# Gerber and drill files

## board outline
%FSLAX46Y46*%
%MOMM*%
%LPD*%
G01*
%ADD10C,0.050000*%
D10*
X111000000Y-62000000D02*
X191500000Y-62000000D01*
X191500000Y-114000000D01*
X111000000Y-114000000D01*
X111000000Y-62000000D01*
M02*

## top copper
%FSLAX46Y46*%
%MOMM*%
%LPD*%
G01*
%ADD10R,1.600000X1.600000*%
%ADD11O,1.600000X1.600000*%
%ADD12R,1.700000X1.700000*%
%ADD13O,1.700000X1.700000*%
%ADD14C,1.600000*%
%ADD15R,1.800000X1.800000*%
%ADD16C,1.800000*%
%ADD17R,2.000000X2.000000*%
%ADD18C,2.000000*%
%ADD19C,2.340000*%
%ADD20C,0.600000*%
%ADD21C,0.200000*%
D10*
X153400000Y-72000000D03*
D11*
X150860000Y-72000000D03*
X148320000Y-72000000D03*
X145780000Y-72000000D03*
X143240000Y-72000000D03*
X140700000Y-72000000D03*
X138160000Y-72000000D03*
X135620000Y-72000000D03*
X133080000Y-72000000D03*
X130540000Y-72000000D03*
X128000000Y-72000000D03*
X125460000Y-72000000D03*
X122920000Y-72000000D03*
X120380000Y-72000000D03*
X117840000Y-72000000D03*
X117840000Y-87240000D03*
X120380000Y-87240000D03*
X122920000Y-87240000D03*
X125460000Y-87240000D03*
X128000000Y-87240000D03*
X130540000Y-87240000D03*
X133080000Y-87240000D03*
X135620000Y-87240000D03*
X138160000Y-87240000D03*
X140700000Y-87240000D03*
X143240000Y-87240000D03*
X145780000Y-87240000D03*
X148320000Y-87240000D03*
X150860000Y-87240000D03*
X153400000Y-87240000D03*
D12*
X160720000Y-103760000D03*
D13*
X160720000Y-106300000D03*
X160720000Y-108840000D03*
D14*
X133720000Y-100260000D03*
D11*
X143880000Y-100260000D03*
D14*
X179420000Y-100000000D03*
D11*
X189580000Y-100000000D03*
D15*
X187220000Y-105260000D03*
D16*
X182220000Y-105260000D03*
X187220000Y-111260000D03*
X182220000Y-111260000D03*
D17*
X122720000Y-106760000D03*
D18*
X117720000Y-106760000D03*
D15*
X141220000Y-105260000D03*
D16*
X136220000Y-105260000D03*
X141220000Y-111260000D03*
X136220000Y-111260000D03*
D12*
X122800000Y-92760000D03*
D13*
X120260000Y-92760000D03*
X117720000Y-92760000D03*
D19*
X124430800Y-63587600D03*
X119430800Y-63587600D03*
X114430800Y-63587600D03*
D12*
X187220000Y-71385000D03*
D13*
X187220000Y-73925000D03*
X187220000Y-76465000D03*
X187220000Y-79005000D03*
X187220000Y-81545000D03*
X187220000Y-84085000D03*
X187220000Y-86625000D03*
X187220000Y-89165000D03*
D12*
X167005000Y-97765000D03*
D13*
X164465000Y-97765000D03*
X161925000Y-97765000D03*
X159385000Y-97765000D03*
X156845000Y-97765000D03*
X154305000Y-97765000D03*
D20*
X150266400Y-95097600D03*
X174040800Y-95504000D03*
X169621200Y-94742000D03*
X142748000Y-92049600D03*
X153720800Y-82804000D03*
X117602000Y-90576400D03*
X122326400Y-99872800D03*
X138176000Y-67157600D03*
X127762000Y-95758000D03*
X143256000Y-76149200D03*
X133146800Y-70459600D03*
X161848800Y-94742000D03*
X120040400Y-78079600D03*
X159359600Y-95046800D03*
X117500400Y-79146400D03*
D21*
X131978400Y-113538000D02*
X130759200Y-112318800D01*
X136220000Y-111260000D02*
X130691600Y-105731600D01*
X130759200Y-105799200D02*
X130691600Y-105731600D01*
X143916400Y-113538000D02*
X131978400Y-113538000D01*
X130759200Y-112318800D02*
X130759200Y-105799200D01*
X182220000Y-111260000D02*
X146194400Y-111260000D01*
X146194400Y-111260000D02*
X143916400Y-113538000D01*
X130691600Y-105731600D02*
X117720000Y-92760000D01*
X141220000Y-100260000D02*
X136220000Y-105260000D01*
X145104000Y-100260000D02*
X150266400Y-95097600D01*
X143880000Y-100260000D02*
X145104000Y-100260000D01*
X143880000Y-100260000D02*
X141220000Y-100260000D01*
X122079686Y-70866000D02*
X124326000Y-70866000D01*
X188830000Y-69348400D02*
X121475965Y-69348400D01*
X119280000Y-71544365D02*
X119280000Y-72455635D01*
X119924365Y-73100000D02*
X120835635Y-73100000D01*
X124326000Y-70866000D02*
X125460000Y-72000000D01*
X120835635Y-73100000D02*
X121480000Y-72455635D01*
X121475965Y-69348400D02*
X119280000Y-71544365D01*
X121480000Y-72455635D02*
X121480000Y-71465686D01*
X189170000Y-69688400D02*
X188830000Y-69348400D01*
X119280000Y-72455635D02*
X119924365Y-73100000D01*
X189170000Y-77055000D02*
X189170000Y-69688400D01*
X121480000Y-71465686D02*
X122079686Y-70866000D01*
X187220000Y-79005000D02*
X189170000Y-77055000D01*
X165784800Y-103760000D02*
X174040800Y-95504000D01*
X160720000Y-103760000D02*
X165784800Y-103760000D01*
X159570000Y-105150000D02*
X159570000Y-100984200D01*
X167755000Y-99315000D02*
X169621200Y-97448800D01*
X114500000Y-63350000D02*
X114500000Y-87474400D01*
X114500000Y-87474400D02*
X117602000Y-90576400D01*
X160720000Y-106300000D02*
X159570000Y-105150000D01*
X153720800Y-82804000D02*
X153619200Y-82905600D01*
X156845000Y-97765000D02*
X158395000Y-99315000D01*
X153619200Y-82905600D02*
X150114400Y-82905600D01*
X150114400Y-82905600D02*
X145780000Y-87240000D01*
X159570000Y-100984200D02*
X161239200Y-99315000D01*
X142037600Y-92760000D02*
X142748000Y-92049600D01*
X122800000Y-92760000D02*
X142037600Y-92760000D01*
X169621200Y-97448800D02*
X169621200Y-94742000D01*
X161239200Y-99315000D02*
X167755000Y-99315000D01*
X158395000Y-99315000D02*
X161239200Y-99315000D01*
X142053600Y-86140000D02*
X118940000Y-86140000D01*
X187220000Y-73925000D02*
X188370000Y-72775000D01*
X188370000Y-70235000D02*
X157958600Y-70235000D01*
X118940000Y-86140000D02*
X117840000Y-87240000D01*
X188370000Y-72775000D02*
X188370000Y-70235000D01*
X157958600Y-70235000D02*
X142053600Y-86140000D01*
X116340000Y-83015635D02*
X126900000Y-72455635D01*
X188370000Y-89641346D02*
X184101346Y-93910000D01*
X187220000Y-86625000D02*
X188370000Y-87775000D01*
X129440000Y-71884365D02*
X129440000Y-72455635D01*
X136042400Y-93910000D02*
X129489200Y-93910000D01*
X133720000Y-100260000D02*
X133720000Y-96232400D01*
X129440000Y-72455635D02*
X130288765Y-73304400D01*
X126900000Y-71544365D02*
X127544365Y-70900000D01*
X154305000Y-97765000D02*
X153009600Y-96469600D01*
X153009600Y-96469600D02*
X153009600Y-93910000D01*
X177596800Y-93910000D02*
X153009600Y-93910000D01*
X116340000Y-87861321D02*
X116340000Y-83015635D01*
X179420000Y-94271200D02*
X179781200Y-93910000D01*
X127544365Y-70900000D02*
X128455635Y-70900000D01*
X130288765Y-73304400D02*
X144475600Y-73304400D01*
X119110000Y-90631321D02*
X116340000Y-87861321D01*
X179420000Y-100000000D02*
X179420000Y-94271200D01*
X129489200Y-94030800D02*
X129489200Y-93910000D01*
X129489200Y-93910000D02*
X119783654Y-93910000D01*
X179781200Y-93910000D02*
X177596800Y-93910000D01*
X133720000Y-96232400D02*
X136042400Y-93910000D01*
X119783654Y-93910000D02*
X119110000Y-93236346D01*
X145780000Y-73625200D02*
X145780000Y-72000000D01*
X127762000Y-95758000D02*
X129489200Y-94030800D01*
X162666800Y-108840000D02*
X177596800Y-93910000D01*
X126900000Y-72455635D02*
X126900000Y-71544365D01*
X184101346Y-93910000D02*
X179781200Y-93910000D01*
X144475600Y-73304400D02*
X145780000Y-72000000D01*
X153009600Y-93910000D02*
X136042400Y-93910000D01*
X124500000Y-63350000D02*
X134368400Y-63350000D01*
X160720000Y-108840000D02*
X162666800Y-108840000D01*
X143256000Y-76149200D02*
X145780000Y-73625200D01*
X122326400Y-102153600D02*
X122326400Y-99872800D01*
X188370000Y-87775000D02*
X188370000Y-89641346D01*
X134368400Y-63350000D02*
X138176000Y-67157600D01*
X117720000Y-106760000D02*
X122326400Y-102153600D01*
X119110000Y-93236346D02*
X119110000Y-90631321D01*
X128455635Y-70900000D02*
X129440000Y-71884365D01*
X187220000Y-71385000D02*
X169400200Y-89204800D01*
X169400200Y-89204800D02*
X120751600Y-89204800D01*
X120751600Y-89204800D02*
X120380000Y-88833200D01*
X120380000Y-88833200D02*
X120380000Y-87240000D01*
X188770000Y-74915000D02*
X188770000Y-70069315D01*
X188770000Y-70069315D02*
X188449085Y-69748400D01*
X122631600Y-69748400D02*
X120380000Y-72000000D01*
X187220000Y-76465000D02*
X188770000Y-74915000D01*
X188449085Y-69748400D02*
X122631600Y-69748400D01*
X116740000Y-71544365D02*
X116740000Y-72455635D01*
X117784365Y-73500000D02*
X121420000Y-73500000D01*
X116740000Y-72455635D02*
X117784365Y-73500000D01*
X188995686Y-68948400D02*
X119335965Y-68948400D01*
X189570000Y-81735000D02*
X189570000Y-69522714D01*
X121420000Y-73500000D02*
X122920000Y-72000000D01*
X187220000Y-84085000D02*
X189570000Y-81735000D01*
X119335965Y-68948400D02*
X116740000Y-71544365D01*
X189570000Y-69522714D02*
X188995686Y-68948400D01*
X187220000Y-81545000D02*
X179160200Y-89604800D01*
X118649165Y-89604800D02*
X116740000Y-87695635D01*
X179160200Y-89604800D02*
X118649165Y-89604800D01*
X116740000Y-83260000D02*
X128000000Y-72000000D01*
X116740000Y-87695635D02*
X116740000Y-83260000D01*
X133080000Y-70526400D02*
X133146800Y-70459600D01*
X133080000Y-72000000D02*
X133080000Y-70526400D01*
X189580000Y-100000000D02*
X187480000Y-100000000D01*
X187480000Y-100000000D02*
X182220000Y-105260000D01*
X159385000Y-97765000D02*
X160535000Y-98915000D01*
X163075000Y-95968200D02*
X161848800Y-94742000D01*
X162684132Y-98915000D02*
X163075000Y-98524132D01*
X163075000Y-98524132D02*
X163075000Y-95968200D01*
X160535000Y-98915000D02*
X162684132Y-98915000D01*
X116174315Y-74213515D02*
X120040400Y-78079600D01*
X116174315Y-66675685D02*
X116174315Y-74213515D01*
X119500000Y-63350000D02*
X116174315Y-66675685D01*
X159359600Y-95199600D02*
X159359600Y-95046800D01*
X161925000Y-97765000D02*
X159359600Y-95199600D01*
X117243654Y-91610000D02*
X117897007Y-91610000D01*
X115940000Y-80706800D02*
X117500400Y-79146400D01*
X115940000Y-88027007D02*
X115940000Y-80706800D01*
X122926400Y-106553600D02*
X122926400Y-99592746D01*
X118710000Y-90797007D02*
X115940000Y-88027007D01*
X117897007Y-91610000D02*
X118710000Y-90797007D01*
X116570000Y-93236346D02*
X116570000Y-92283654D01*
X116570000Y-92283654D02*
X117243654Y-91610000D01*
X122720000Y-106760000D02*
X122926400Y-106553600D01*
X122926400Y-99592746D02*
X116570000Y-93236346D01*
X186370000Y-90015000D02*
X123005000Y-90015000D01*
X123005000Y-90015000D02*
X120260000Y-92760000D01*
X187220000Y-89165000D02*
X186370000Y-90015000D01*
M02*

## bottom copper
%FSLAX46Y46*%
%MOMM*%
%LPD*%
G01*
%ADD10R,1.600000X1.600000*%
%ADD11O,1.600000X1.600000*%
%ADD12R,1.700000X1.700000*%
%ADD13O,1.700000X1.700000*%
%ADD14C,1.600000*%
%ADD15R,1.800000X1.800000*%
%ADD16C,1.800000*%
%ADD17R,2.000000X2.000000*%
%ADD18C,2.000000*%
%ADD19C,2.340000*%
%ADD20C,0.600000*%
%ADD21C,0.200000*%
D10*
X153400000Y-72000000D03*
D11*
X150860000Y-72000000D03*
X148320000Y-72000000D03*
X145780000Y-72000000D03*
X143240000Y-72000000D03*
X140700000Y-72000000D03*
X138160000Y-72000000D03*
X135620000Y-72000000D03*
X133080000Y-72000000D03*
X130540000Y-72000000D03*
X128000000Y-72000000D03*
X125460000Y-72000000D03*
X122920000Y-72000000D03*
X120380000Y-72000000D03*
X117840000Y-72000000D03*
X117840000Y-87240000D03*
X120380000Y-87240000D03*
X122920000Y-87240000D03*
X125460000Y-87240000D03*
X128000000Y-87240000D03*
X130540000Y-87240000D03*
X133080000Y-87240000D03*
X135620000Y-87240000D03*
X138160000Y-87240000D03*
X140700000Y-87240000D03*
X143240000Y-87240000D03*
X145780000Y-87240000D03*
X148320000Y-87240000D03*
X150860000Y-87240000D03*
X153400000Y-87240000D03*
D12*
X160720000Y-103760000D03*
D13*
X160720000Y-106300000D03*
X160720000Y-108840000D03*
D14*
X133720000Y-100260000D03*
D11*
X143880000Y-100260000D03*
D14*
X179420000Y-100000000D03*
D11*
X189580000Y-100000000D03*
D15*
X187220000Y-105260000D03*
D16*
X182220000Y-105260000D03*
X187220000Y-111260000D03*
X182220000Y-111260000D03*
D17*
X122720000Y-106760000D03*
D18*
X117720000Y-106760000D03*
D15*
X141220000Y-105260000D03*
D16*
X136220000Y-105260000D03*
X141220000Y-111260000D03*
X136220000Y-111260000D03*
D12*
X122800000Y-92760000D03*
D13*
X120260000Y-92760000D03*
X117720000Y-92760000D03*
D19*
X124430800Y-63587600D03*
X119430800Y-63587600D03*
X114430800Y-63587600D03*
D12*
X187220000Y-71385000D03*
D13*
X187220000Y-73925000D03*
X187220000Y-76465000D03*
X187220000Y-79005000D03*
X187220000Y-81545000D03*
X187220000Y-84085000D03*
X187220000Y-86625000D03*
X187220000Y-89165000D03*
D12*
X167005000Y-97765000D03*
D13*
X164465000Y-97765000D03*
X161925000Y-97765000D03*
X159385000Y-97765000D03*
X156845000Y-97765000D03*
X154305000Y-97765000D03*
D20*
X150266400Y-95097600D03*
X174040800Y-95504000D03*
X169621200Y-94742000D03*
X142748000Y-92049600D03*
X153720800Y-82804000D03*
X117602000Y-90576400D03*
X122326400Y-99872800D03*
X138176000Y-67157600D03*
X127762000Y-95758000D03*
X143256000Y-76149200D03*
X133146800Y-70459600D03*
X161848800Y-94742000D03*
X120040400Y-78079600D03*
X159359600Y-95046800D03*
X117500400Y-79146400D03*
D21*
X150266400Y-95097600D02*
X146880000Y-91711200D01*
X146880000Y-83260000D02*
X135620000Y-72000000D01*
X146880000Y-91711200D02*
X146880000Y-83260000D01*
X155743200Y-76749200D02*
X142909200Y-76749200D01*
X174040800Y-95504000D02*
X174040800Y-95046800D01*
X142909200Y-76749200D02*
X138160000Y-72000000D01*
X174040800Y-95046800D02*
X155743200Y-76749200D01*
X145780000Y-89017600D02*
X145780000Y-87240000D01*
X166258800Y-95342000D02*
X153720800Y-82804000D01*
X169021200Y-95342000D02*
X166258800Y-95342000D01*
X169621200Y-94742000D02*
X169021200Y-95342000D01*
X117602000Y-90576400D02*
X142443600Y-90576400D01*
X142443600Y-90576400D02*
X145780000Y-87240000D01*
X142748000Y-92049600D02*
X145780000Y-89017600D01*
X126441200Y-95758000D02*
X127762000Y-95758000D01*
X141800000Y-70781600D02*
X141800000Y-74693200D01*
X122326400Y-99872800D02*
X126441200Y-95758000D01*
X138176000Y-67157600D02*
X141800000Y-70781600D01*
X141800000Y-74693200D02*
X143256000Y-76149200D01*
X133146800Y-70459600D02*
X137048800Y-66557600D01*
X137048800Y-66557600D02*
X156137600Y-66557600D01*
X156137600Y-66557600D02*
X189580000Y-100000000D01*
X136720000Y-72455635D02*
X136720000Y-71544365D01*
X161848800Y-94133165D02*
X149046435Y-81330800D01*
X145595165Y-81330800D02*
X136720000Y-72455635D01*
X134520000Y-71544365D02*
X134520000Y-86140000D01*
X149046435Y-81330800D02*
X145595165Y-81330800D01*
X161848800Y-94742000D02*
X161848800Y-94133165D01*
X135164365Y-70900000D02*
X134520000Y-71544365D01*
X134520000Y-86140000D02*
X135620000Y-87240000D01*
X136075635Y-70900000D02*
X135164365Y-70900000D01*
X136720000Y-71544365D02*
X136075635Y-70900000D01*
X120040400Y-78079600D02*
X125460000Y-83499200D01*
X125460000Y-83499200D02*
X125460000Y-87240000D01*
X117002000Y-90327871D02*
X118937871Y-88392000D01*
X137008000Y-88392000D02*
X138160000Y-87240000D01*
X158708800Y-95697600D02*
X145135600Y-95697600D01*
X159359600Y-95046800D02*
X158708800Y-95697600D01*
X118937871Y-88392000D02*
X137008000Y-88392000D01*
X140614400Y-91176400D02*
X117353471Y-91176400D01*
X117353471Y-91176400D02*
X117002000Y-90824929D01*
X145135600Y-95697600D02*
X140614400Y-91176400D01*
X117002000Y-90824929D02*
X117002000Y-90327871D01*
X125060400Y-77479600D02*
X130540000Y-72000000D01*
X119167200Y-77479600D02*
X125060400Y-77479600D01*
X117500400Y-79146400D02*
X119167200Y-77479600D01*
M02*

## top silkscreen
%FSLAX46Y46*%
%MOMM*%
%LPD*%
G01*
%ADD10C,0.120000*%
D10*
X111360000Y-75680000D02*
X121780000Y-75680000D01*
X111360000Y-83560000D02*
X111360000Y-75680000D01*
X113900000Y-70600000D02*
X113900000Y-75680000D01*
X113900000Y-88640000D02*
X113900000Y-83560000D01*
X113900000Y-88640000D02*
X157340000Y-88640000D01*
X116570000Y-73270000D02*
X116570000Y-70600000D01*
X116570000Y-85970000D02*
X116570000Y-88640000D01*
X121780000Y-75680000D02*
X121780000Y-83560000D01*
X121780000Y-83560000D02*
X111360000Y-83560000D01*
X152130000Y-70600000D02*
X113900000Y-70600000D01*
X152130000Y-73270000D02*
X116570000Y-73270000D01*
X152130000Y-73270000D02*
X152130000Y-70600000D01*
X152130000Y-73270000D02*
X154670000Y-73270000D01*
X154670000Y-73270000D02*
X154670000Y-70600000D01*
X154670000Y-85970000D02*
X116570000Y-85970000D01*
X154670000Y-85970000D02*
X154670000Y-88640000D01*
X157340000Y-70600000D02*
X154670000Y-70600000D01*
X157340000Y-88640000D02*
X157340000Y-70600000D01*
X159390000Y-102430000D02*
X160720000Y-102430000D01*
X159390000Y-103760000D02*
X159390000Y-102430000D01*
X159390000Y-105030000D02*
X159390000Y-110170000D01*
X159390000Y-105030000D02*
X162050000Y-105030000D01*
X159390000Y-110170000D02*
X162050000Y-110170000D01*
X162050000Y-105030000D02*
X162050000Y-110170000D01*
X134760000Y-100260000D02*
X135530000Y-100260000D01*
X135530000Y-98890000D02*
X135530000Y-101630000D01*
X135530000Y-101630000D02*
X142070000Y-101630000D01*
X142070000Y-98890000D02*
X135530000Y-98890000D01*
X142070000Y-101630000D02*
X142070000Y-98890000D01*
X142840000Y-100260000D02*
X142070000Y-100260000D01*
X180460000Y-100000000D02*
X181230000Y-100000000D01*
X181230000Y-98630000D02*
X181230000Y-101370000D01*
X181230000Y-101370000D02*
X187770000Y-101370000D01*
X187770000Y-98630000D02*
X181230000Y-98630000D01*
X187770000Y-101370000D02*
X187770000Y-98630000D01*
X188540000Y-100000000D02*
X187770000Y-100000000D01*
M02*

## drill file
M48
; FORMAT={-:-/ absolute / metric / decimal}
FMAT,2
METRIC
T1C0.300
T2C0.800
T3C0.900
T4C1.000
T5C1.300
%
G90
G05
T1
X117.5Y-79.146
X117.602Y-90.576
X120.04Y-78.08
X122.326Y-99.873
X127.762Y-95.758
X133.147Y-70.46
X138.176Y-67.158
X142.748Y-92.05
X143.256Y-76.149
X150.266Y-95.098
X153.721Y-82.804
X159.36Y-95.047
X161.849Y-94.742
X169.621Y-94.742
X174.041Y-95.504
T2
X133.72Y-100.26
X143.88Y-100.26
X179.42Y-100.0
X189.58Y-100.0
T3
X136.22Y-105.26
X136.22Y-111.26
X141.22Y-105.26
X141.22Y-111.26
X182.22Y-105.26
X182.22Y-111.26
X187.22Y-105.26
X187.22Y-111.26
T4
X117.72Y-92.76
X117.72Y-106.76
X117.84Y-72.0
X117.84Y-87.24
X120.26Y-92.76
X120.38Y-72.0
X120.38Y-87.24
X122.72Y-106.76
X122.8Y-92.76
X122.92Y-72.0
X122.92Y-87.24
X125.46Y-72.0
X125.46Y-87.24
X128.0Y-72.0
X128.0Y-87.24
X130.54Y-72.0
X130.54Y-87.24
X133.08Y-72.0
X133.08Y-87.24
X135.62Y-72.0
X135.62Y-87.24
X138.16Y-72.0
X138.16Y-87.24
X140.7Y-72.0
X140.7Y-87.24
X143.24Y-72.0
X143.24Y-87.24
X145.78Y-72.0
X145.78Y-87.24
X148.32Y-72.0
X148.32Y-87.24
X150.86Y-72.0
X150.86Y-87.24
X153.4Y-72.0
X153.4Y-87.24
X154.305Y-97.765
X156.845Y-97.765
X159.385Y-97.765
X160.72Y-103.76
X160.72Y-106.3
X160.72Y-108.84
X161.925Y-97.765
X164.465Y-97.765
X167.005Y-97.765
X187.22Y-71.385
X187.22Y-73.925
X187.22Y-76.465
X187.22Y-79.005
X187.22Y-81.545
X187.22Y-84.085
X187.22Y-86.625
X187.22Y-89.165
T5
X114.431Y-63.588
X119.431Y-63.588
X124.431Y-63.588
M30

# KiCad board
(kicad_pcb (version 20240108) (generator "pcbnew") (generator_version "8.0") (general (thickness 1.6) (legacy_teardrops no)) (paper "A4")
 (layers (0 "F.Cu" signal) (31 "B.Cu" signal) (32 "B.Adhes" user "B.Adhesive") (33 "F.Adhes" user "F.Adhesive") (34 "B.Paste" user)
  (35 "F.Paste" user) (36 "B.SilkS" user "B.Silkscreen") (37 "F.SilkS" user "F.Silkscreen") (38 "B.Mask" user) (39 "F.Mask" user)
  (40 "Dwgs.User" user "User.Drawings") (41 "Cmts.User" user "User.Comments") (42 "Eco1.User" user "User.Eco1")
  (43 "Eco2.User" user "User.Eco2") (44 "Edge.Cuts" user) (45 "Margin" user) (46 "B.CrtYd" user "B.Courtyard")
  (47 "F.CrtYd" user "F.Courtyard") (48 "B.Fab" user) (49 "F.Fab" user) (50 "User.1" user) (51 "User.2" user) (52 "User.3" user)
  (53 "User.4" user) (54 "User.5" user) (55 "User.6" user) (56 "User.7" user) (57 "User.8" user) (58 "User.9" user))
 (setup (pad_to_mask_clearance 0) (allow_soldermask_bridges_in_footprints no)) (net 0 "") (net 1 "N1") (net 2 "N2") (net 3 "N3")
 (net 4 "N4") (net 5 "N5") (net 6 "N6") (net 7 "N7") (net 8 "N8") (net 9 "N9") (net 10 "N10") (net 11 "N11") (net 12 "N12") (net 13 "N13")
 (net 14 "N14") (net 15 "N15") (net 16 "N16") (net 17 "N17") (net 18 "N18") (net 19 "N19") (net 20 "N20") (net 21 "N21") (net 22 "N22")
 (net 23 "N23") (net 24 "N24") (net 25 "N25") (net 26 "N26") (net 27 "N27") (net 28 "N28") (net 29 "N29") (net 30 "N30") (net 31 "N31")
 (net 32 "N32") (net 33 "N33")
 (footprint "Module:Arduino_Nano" (layer "F.Cu") (at 153.4 72 -90)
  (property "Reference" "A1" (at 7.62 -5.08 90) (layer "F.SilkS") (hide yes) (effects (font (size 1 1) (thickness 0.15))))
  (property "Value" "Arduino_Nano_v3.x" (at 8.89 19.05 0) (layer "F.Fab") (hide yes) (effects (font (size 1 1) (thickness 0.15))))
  (fp_line (start 3.68 42.04) (end 3.68 31.62) (stroke (width 0.12) (type solid)) (layer "F.SilkS"))
  (fp_line (start 11.56 42.04) (end 3.68 42.04) (stroke (width 0.12) (type solid)) (layer "F.SilkS"))
  (fp_line (start -1.4 39.5) (end 3.68 39.5) (stroke (width 0.12) (type solid)) (layer "F.SilkS"))
  (fp_line (start 16.64 39.5) (end 11.56 39.5) (stroke (width 0.12) (type solid)) (layer "F.SilkS"))
  (fp_line (start 16.64 39.5) (end 16.64 -3.94) (stroke (width 0.12) (type solid)) (layer "F.SilkS"))
  (fp_line (start 1.27 36.83) (end -1.4 36.83) (stroke (width 0.12) (type solid)) (layer "F.SilkS"))
  (fp_line (start 13.97 36.83) (end 16.64 36.83) (stroke (width 0.12) (type solid)) (layer "F.SilkS"))
  (fp_line (start 3.68 31.62) (end 11.56 31.62) (stroke (width 0.12) (type solid)) (layer "F.SilkS"))
  (fp_line (start 11.56 31.62) (end 11.56 42.04) (stroke (width 0.12) (type solid)) (layer "F.SilkS"))
  (fp_line (start -1.4 1.27) (end -1.4 39.5) (stroke (width 0.12) (type solid)) (layer "F.SilkS"))
  (fp_line (start 1.27 1.27) (end 1.27 36.83) (stroke (width 0.12) (type solid)) (layer "F.SilkS"))
  (fp_line (start 1.27 1.27) (end -1.4 1.27) (stroke (width 0.12) (type solid)) (layer "F.SilkS"))
  (fp_line (start 1.27 1.27) (end 1.27 -1.27) (stroke (width 0.12) (type solid)) (layer "F.SilkS"))
  (fp_line (start 1.27 -1.27) (end -1.4 -1.27) (stroke (width 0.12) (type solid)) (layer "F.SilkS"))
  (fp_line (start 13.97 -1.27) (end 13.97 36.83) (stroke (width 0.12) (type solid)) (layer "F.SilkS"))
  (fp_line (start 13.97 -1.27) (end 16.64 -1.27) (stroke (width 0.12) (type solid)) (layer "F.SilkS"))
  (fp_line (start -1.4 -3.94) (end -1.4 -1.27) (stroke (width 0.12) (type solid)) (layer "F.SilkS"))
  (fp_line (start 16.64 -3.94) (end -1.4 -3.94) (stroke (width 0.12) (type solid)) (layer "F.SilkS"))
  (pad "1" thru_hole rect (at 0 0 270) (size 1.6 1.6) (drill 1) (layers "*.Cu" "*.Mask") (remove_unused_layers no) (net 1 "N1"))
  (pad "2" thru_hole oval (at 0 2.54 270) (size 1.6 1.6) (drill 1) (layers "*.Cu" "*.Mask") (remove_unused_layers no) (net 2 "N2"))
  (pad "3" thru_hole oval (at 0 5.08 270) (size 1.6 1.6) (drill 1) (layers "*.Cu" "*.Mask") (remove_unused_layers no) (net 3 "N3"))
  (pad "4" thru_hole oval (at 0 7.62 270) (size 1.6 1.6) (drill 1) (layers "*.Cu" "*.Mask") (remove_unused_layers no) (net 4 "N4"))
  (pad "5" thru_hole oval (at 0 10.16 270) (size 1.6 1.6) (drill 1) (layers "*.Cu" "*.Mask") (remove_unused_layers no) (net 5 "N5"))
  (pad "6" thru_hole oval (at 0 12.7 270) (size 1.6 1.6) (drill 1) (layers "*.Cu" "*.Mask") (remove_unused_layers no) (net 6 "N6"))
  (pad "7" thru_hole oval (at 0 15.24 270) (size 1.6 1.6) (drill 1) (layers "*.Cu" "*.Mask") (remove_unused_layers no) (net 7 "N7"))
  (pad "8" thru_hole oval (at 0 17.78 270) (size 1.6 1.6) (drill 1) (layers "*.Cu" "*.Mask") (remove_unused_layers no) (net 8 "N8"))
  (pad "9" thru_hole oval (at 0 20.32 270) (size 1.6 1.6) (drill 1) (layers "*.Cu" "*.Mask") (remove_unused_layers no) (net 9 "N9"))
  (pad "10" thru_hole oval (at 0 22.86 270) (size 1.6 1.6) (drill 1) (layers "*.Cu" "*.Mask") (remove_unused_layers no) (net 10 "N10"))
  (pad "11" thru_hole oval (at 0 25.4 270) (size 1.6 1.6) (drill 1) (layers "*.Cu" "*.Mask") (remove_unused_layers no) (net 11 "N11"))
  (pad "12" thru_hole oval (at 0 27.94 270) (size 1.6 1.6) (drill 1) (layers "*.Cu" "*.Mask") (remove_unused_layers no) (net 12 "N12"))
  (pad "13" thru_hole oval (at 0 30.48 270) (size 1.6 1.6) (drill 1) (layers "*.Cu" "*.Mask") (remove_unused_layers no) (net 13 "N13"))
  (pad "14" thru_hole oval (at 0 33.02 270) (size 1.6 1.6) (drill 1) (layers "*.Cu" "*.Mask") (remove_unused_layers no) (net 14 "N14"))
  (pad "15" thru_hole oval (at 0 35.56 270) (size 1.6 1.6) (drill 1) (layers "*.Cu" "*.Mask") (remove_unused_layers no) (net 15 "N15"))
  (pad "16" thru_hole oval (at 15.24 35.56 270) (size 1.6 1.6) (drill 1) (layers "*.Cu" "*.Mask") (remove_unused_layers no) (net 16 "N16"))
  (pad "17" thru_hole oval (at 15.24 33.02 270) (size 1.6 1.6) (drill 1) (layers "*.Cu" "*.Mask") (remove_unused_layers no) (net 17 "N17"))
  (pad "18" thru_hole oval (at 15.24 30.48 270) (size 1.6 1.6) (drill 1) (layers "*.Cu" "*.Mask") (remove_unused_layers no) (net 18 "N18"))
  (pad "19" thru_hole oval (at 15.24 27.94 270) (size 1.6 1.6) (drill 1) (layers "*.Cu" "*.Mask") (remove_unused_layers no) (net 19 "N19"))
  (pad "20" thru_hole oval (at 15.24 25.4 270) (size 1.6 1.6) (drill 1) (layers "*.Cu" "*.Mask") (remove_unused_layers no) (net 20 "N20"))
  (pad "21" thru_hole oval (at 15.24 22.86 270) (size 1.6 1.6) (drill 1) (layers "*.Cu" "*.Mask") (remove_unused_layers no) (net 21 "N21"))
  (pad "22" thru_hole oval (at 15.24 20.32 270) (size 1.6 1.6) (drill 1) (layers "*.Cu" "*.Mask") (remove_unused_layers no) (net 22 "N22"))
  (pad "23" thru_hole oval (at 15.24 17.78 270) (size 1.6 1.6) (drill 1) (layers "*.Cu" "*.Mask") (remove_unused_layers no) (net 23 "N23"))
  (pad "24" thru_hole oval (at 15.24 15.24 270) (size 1.6 1.6) (drill 1) (layers "*.Cu" "*.Mask") (remove_unused_layers no) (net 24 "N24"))
  (pad "25" thru_hole oval (at 15.24 12.7 270) (size 1.6 1.6) (drill 1) (layers "*.Cu" "*.Mask") (remove_unused_layers no) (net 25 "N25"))
  (pad "26" thru_hole oval (at 15.24 10.16 270) (size 1.6 1.6) (drill 1) (layers "*.Cu" "*.Mask") (remove_unused_layers no) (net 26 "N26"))
  (pad "27" thru_hole oval (at 15.24 7.62 270) (size 1.6 1.6) (drill 1) (layers "*.Cu" "*.Mask") (remove_unused_layers no) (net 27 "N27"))
  (pad "28" thru_hole oval (at 15.24 5.08 270) (size 1.6 1.6) (drill 1) (layers "*.Cu" "*.Mask") (remove_unused_layers no) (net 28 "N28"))
  (pad "29" thru_hole oval (at 15.24 2.54 270) (size 1.6 1.6) (drill 1) (layers "*.Cu" "*.Mask") (remove_unused_layers no) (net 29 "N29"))
  (pad "30" thru_hole oval (at 15.24 0 270) (size 1.6 1.6) (drill 1) (layers "*.Cu" "*.Mask") (remove_unused_layers no) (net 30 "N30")))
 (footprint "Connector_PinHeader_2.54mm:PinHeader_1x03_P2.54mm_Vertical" (layer "F.Cu") (at 160.72 103.76)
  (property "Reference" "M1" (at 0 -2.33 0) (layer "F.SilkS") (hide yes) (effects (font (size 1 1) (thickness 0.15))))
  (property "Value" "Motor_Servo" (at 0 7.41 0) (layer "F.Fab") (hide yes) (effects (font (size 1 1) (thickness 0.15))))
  (fp_line (start -1.33 -1.33) (end 0 -1.33) (stroke (width 0.12) (type solid)) (layer "F.SilkS"))
  (fp_line (start -1.33 0) (end -1.33 -1.33) (stroke (width 0.12) (type solid)) (layer "F.SilkS"))
  (fp_line (start -1.33 1.27) (end -1.33 6.41) (stroke (width 0.12) (type solid)) (layer "F.SilkS"))
  (fp_line (start -1.33 1.27) (end 1.33 1.27) (stroke (width 0.12) (type solid)) (layer "F.SilkS"))
  (fp_line (start -1.33 6.41) (end 1.33 6.41) (stroke (width 0.12) (type solid)) (layer "F.SilkS"))
  (fp_line (start 1.33 1.27) (end 1.33 6.41) (stroke (width 0.12) (type solid)) (layer "F.SilkS"))
  (pad "1" thru_hole rect (at 0 0) (size 1.7 1.7) (drill 1) (layers "*.Cu" "*.Mask") (remove_unused_layers no) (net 7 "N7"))
  (pad "2" thru_hole oval (at 0 2.54) (size 1.7 1.7) (drill 1) (layers "*.Cu" "*.Mask") (remove_unused_layers no) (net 27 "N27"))
  (pad "3" thru_hole oval (at 0 5.08) (size 1.7 1.7) (drill 1) (layers "*.Cu" "*.Mask") (remove_unused_layers no) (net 4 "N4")))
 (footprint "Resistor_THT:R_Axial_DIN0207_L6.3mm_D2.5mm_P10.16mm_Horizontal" (layer "F.Cu") (at 133.72 100.26)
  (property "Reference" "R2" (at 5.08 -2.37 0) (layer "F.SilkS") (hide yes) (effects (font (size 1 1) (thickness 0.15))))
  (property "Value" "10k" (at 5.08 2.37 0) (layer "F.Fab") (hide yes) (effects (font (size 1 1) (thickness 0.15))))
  (fp_line (start 1.04 0) (end 1.81 0) (stroke (width 0.12) (type solid)) (layer "F.SilkS"))
  (fp_line (start 1.81 -1.37) (end 1.81 1.37) (stroke (width 0.12) (type solid)) (layer "F.SilkS"))
  (fp_line (start 1.81 1.37) (end 8.35 1.37) (stroke (width 0.12) (type solid)) (layer "F.SilkS"))
  (fp_line (start 8.35 -1.37) (end 1.81 -1.37) (stroke (width 0.12) (type solid)) (layer "F.SilkS"))
  (fp_line (start 8.35 1.37) (end 8.35 -1.37) (stroke (width 0.12) (type solid)) (layer "F.SilkS"))
  (fp_line (start 9.12 0) (end 8.35 0) (stroke (width 0.12) (type solid)) (layer "F.SilkS"))
  (pad "1" thru_hole circle (at 0 0) (size 1.6 1.6) (drill 0.8) (layers "*.Cu" "*.Mask") (remove_unused_layers no) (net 4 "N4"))
  (pad "2" thru_hole oval (at 10.16 0) (size 1.6 1.6) (drill 0.8) (layers "*.Cu" "*.Mask") (remove_unused_layers no) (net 8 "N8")))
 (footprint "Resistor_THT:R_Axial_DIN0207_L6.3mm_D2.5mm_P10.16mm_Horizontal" (layer "F.Cu") (at 179.42 100)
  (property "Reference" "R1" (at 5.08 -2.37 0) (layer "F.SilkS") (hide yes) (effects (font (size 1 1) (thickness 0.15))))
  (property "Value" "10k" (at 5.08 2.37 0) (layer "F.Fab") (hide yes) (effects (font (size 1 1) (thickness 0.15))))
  (fp_line (start 1.04 0) (end 1.81 0) (stroke (width 0.12) (type solid)) (layer "F.SilkS"))
  (fp_line (start 1.81 -1.37) (end 1.81 1.37) (stroke (width 0.12) (type solid)) (layer "F.SilkS"))
  (fp_line (start 1.81 1.37) (end 8.35 1.37) (stroke (width 0.12) (type solid)) (layer "F.SilkS"))
  (fp_line (start 8.35 -1.37) (end 1.81 -1.37) (stroke (width 0.12) (type solid)) (layer "F.SilkS"))
  (fp_line (start 8.35 1.37) (end 8.35 -1.37) (stroke (width 0.12) (type solid)) (layer "F.SilkS"))
  (fp_line (start 9.12 0) (end 8.35 0) (stroke (width 0.12) (type solid)) (layer "F.SilkS"))
  (pad "1" thru_hole circle (at 0 0) (size 1.6 1.6) (drill 0.8) (layers "*.Cu" "*.Mask") (remove_unused_layers no) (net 4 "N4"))
  (pad "2" thru_hole oval (at 10.16 0) (size 1.6 1.6) (drill 0.8) (layers "*.Cu" "*.Mask") (remove_unused_layers no) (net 9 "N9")))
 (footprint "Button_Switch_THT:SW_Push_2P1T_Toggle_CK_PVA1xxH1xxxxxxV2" (layer "B.Cu") (at 187.22 105.26 180)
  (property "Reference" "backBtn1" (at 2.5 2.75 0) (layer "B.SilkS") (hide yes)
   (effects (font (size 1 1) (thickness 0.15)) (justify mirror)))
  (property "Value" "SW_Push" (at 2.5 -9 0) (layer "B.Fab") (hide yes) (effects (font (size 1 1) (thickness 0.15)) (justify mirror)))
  (pad "1" thru_hole rect (at 0 0 180) (size 1.8 1.8) (drill 0.9) (layers "*.Cu" "*.Mask") (remove_unused_layers no) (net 27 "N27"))
  (pad "2" thru_hole circle (at 5 0 180) (size 1.8 1.8) (drill 0.9) (layers "*.Cu" "*.Mask") (remove_unused_layers no) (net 9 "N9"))
  (pad "3" thru_hole circle (at 0 -6 180) (size 1.8 1.8) (drill 0.9) (layers "*.Cu" "*.Mask") (remove_unused_layers no))
  (pad "4" thru_hole circle (at 5 -6 180) (size 1.8 1.8) (drill 0.9) (layers "*.Cu" "*.Mask") (remove_unused_layers no)))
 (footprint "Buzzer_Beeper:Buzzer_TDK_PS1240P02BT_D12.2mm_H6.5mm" (layer "B.Cu") (at 122.72 106.76 180)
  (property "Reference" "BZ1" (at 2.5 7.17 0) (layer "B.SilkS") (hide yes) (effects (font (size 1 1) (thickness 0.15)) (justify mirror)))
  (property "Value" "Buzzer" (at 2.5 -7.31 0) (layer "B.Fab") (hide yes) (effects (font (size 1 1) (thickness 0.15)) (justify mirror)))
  (pad "1" thru_hole rect (at 0 0 180) (size 2 2) (drill 1) (layers "*.Cu" "*.Mask") (remove_unused_layers no) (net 10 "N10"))
  (pad "2" thru_hole circle (at 5 0 180) (size 2 2) (drill 1) (layers "*.Cu" "*.Mask") (remove_unused_layers no) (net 4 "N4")))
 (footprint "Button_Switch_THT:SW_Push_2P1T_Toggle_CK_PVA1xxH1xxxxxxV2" (layer "B.Cu") (at 141.22 105.26 180)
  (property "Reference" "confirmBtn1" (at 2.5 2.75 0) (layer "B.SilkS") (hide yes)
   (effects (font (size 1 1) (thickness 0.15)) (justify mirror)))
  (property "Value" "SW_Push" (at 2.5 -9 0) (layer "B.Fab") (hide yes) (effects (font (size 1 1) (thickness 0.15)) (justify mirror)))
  (pad "1" thru_hole rect (at 0 0 180) (size 1.8 1.8) (drill 0.9) (layers "*.Cu" "*.Mask") (remove_unused_layers no) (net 27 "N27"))
  (pad "2" thru_hole circle (at 5 0 180) (size 1.8 1.8) (drill 0.9) (layers "*.Cu" "*.Mask") (remove_unused_layers no) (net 8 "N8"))
  (pad "3" thru_hole circle (at 0 -6 180) (size 1.8 1.8) (drill 0.9) (layers "*.Cu" "*.Mask") (remove_unused_layers no))
  (pad "4" thru_hole circle (at 5 -6 180) (size 1.8 1.8) (drill 0.9) (layers "*.Cu" "*.Mask") (remove_unused_layers no)))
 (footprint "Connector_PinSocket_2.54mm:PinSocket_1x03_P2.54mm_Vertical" (layer "B.Cu") (at 122.8 92.76 90)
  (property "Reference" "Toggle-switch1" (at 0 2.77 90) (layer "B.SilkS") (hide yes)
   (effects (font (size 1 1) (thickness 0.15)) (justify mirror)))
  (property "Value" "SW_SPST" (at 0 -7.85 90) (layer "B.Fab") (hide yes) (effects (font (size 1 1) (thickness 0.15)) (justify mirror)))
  (pad "1" thru_hole rect (at 0 0 90) (size 1.7 1.7) (drill 1) (layers "*.Cu" "*.Mask") (remove_unused_layers no) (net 27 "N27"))
  (pad "2" thru_hole oval (at 0 -2.54 90) (size 1.7 1.7) (drill 1) (layers "*.Cu" "*.Mask") (remove_unused_layers no) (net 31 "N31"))
  (pad "3" thru_hole oval (at 0 -5.08 90) (size 1.7 1.7) (drill 1) (layers "*.Cu" "*.Mask") (remove_unused_layers no)))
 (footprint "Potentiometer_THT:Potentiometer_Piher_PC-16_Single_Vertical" (layer "B.Cu") (at 124.4308 63.5876 -90)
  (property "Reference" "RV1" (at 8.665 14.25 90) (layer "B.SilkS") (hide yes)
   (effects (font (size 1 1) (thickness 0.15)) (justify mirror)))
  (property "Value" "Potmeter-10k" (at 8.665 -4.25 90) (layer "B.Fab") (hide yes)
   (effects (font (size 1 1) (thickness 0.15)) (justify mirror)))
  (pad "1" thru_hole circle (at 0 0 270) (size 2.34 2.34) (drill 1.3) (layers "*.Cu" "*.Mask") (remove_unused_layers no) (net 4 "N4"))
  (pad "2" thru_hole circle (at 0 5 270) (size 2.34 2.34) (drill 1.3) (layers "*.Cu" "*.Mask") (remove_unused_layers no) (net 19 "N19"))
  (pad "3" thru_hole circle (at 0 10 270) (size 2.34 2.34) (drill 1.3) (layers "*.Cu" "*.Mask") (remove_unused_layers no) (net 27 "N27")))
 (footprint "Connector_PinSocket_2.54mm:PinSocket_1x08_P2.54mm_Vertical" (layer "B.Cu") (at 187.22 71.385 180)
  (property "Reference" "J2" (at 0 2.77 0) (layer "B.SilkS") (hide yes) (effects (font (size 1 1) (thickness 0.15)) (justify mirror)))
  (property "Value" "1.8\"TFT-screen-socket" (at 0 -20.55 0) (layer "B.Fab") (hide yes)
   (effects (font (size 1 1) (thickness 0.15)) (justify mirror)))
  (pad "1" thru_hole rect (at 0 0 180) (size 1.7 1.7) (drill 1) (layers "*.Cu" "*.Mask") (remove_unused_layers no) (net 17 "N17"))
  (pad "2" thru_hole oval (at 0 -2.54 180) (size 1.7 1.7) (drill 1) (layers "*.Cu" "*.Mask") (remove_unused_layers no) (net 16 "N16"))
  (pad "3" thru_hole oval (at 0 -5.08 180) (size 1.7 1.7) (drill 1) (layers "*.Cu" "*.Mask") (remove_unused_layers no) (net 14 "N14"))
  (pad "4" thru_hole oval (at 0 -7.62 180) (size 1.7 1.7) (drill 1) (layers "*.Cu" "*.Mask") (remove_unused_layers no) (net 12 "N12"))
  (pad "5" thru_hole oval (at 0 -10.16 180) (size 1.7 1.7) (drill 1) (layers "*.Cu" "*.Mask") (remove_unused_layers no) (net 11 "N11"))
  (pad "6" thru_hole oval (at 0 -12.7 180) (size 1.7 1.7) (drill 1) (layers "*.Cu" "*.Mask") (remove_unused_layers no) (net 13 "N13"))
  (pad "7" thru_hole oval (at 0 -15.24 180) (size 1.7 1.7) (drill 1) (layers "*.Cu" "*.Mask") (remove_unused_layers no) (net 4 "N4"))
  (pad "8" thru_hole oval (at 0 -17.78 180) (size 1.7 1.7) (drill 1) (layers "*.Cu" "*.Mask") (remove_unused_layers no) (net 31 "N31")))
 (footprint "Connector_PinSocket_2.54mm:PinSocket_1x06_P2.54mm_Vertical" (layer "B.Cu") (at 167.005 97.765 90)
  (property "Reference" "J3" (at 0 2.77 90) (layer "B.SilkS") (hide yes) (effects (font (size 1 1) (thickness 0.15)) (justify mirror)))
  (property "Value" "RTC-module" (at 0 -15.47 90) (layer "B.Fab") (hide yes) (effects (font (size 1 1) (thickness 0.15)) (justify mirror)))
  (pad "1" thru_hole rect (at 0 0 90) (size 1.7 1.7) (drill 1) (layers "*.Cu" "*.Mask") (remove_unused_layers no) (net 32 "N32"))
  (pad "2" thru_hole oval (at 0 -2.54 90) (size 1.7 1.7) (drill 1) (layers "*.Cu" "*.Mask") (remove_unused_layers no) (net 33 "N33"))
  (pad "3" thru_hole oval (at 0 -5.08 90) (size 1.7 1.7) (drill 1) (layers "*.Cu" "*.Mask") (remove_unused_layers no) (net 24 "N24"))
  (pad "4" thru_hole oval (at 0 -7.62 90) (size 1.7 1.7) (drill 1) (layers "*.Cu" "*.Mask") (remove_unused_layers no) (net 23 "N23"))
  (pad "5" thru_hole oval (at 0 -10.16 90) (size 1.7 1.7) (drill 1) (layers "*.Cu" "*.Mask") (remove_unused_layers no) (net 27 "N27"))
  (pad "6" thru_hole oval (at 0 -12.7 90) (size 1.7 1.7) (drill 1) (layers "*.Cu" "*.Mask") (remove_unused_layers no) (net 4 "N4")))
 (gr_rect (start 111 62) (end 191.5 114) (stroke (width 0.05) (type default)) (fill none) (layer "Edge.Cuts"))
 (segment (start 131.9784 113.538) (end 130.7592 112.3188) (width 0.2) (layer "F.Cu") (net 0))
 (segment (start 136.22 111.26) (end 130.6916 105.7316) (width 0.2) (layer "F.Cu") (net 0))
 (segment (start 130.7592 105.7992) (end 130.6916 105.7316) (width 0.2) (layer "F.Cu") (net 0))
 (segment (start 143.9164 113.538) (end 131.9784 113.538) (width 0.2) (layer "F.Cu") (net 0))
 (segment (start 130.7592 112.3188) (end 130.7592 105.7992) (width 0.2) (layer "F.Cu") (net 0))
 (segment (start 182.22 111.26) (end 146.1944 111.26) (width 0.2) (layer "F.Cu") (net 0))
 (segment (start 146.1944 111.26) (end 143.9164 113.538) (width 0.2) (layer "F.Cu") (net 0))
 (segment (start 130.6916 105.7316) (end 117.72 92.76) (width 0.2) (layer "F.Cu") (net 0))
 (segment (start 141.22 100.26) (end 136.22 105.26) (width 0.2) (layer "F.Cu") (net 8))
 (segment (start 145.104 100.26) (end 150.2664 95.0976) (width 0.2) (layer "F.Cu") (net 8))
 (segment (start 143.88 100.26) (end 145.104 100.26) (width 0.2) (layer "F.Cu") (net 8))
 (segment (start 143.88 100.26) (end 141.22 100.26) (width 0.2) (layer "F.Cu") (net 8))
 (via (at 150.2664 95.0976) (size 0.6) (drill 0.3) (layers "F.Cu" "B.Cu") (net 8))
 (segment (start 150.2664 95.0976) (end 146.88 91.7112) (width 0.2) (layer "B.Cu") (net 8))
 (segment (start 146.88 83.26) (end 135.62 72) (width 0.2) (layer "B.Cu") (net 8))
 (segment (start 146.88 91.7112) (end 146.88 83.26) (width 0.2) (layer "B.Cu") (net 8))
 (segment (start 122.079686 70.866) (end 124.326 70.866) (width 0.2) (layer "F.Cu") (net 12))
 (segment (start 188.83 69.3484) (end 121.475965 69.3484) (width 0.2) (layer "F.Cu") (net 12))
 (segment (start 119.28 71.544365) (end 119.28 72.455635) (width 0.2) (layer "F.Cu") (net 12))
 (segment (start 119.924365 73.1) (end 120.835635 73.1) (width 0.2) (layer "F.Cu") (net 12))
 (segment (start 124.326 70.866) (end 125.46 72) (width 0.2) (layer "F.Cu") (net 12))
 (segment (start 120.835635 73.1) (end 121.48 72.455635) (width 0.2) (layer "F.Cu") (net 12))
 (segment (start 121.475965 69.3484) (end 119.28 71.544365) (width 0.2) (layer "F.Cu") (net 12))
 (segment (start 121.48 72.455635) (end 121.48 71.465686) (width 0.2) (layer "F.Cu") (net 12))
 (segment (start 189.17 69.6884) (end 188.83 69.3484) (width 0.2) (layer "F.Cu") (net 12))
 (segment (start 119.28 72.455635) (end 119.924365 73.1) (width 0.2) (layer "F.Cu") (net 12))
 (segment (start 189.17 77.055) (end 189.17 69.6884) (width 0.2) (layer "F.Cu") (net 12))
 (segment (start 121.48 71.465686) (end 122.079686 70.866) (width 0.2) (layer "F.Cu") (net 12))
 (segment (start 187.22 79.005) (end 189.17 77.055) (width 0.2) (layer "F.Cu") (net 12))
 (segment (start 165.7848 103.76) (end 174.0408 95.504) (width 0.2) (layer "F.Cu") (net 7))
 (segment (start 160.72 103.76) (end 165.7848 103.76) (width 0.2) (layer "F.Cu") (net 7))
 (via (at 174.0408 95.504) (size 0.6) (drill 0.3) (layers "F.Cu" "B.Cu") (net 7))
 (segment (start 155.7432 76.7492) (end 142.9092 76.7492) (width 0.2) (layer "B.Cu") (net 7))
 (segment (start 174.0408 95.504) (end 174.0408 95.0468) (width 0.2) (layer "B.Cu") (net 7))
 (segment (start 142.9092 76.7492) (end 138.16 72) (width 0.2) (layer "B.Cu") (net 7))
 (segment (start 174.0408 95.0468) (end 155.7432 76.7492) (width 0.2) (layer "B.Cu") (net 7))
 (segment (start 159.57 105.15) (end 159.57 100.9842) (width 0.2) (layer "F.Cu") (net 27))
 (segment (start 167.755 99.315) (end 169.6212 97.4488) (width 0.2) (layer "F.Cu") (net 27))
 (segment (start 114.5 63.35) (end 114.5 87.4744) (width 0.2) (layer "F.Cu") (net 27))
 (segment (start 114.5 87.4744) (end 117.602 90.5764) (width 0.2) (layer "F.Cu") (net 27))
 (segment (start 160.72 106.3) (end 159.57 105.15) (width 0.2) (layer "F.Cu") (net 27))
 (segment (start 153.7208 82.804) (end 153.6192 82.9056) (width 0.2) (layer "F.Cu") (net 27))
 (segment (start 156.845 97.765) (end 158.395 99.315) (width 0.2) (layer "F.Cu") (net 27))
 (segment (start 153.6192 82.9056) (end 150.1144 82.9056) (width 0.2) (layer "F.Cu") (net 27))
 (segment (start 150.1144 82.9056) (end 145.78 87.24) (width 0.2) (layer "F.Cu") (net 27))
 (segment (start 159.57 100.9842) (end 161.2392 99.315) (width 0.2) (layer "F.Cu") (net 27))
 (segment (start 142.0376 92.76) (end 142.748 92.0496) (width 0.2) (layer "F.Cu") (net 27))
 (segment (start 122.8 92.76) (end 142.0376 92.76) (width 0.2) (layer "F.Cu") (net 27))
 (segment (start 169.6212 97.4488) (end 169.6212 94.742) (width 0.2) (layer "F.Cu") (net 27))
 (segment (start 161.2392 99.315) (end 167.755 99.315) (width 0.2) (layer "F.Cu") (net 27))
 (segment (start 158.395 99.315) (end 161.2392 99.315) (width 0.2) (layer "F.Cu") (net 27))
 (via (at 169.6212 94.742) (size 0.6) (drill 0.3) (layers "F.Cu" "B.Cu") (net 27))
 (via (at 142.748 92.0496) (size 0.6) (drill 0.3) (layers "F.Cu" "B.Cu") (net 27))
 (via (at 153.7208 82.804) (size 0.6) (drill 0.3) (layers "F.Cu" "B.Cu") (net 27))
 (via (at 117.602 90.5764) (size 0.6) (drill 0.3) (layers "F.Cu" "B.Cu") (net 27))
 (segment (start 145.78 89.0176) (end 145.78 87.24) (width 0.2) (layer "B.Cu") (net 27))
 (segment (start 166.2588 95.342) (end 153.7208 82.804) (width 0.2) (layer "B.Cu") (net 27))
 (segment (start 169.0212 95.342) (end 166.2588 95.342) (width 0.2) (layer "B.Cu") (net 27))
 (segment (start 169.6212 94.742) (end 169.0212 95.342) (width 0.2) (layer "B.Cu") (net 27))
 (segment (start 117.602 90.5764) (end 142.4436 90.5764) (width 0.2) (layer "B.Cu") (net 27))
 (segment (start 142.4436 90.5764) (end 145.78 87.24) (width 0.2) (layer "B.Cu") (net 27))
 (segment (start 142.748 92.0496) (end 145.78 89.0176) (width 0.2) (layer "B.Cu") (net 27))
 (segment (start 142.0536 86.14) (end 118.94 86.14) (width 0.2) (layer "F.Cu") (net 16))
 (segment (start 187.22 73.925) (end 188.37 72.775) (width 0.2) (layer "F.Cu") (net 16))
 (segment (start 188.37 70.235) (end 157.9586 70.235) (width 0.2) (layer "F.Cu") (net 16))
 (segment (start 118.94 86.14) (end 117.84 87.24) (width 0.2) (layer "F.Cu") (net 16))
 (segment (start 188.37 72.775) (end 188.37 70.235) (width 0.2) (layer "F.Cu") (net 16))
 (segment (start 157.9586 70.235) (end 142.0536 86.14) (width 0.2) (layer "F.Cu") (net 16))
 (segment (start 116.34 83.015635) (end 126.9 72.455635) (width 0.2) (layer "F.Cu") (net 4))
 (segment (start 188.37 89.641346) (end 184.101346 93.91) (width 0.2) (layer "F.Cu") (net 4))
 (segment (start 187.22 86.625) (end 188.37 87.775) (width 0.2) (layer "F.Cu") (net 4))
 (segment (start 129.44 71.884365) (end 129.44 72.455635) (width 0.2) (layer "F.Cu") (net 4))
 (segment (start 136.0424 93.91) (end 129.4892 93.91) (width 0.2) (layer "F.Cu") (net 4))
 (segment (start 133.72 100.26) (end 133.72 96.2324) (width 0.2) (layer "F.Cu") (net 4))
 (segment (start 129.44 72.455635) (end 130.288765 73.3044) (width 0.2) (layer "F.Cu") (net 4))
 (segment (start 126.9 71.544365) (end 127.544365 70.9) (width 0.2) (layer "F.Cu") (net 4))
 (segment (start 154.305 97.765) (end 153.0096 96.4696) (width 0.2) (layer "F.Cu") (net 4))
 (segment (start 153.0096 96.4696) (end 153.0096 93.91) (width 0.2) (layer "F.Cu") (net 4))
 (segment (start 177.5968 93.91) (end 153.0096 93.91) (width 0.2) (layer "F.Cu") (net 4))
 (segment (start 116.34 87.861321) (end 116.34 83.015635) (width 0.2) (layer "F.Cu") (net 4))
 (segment (start 179.42 94.2712) (end 179.7812 93.91) (width 0.2) (layer "F.Cu") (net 4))
 (segment (start 127.544365 70.9) (end 128.455635 70.9) (width 0.2) (layer "F.Cu") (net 4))
 (segment (start 130.288765 73.3044) (end 144.4756 73.3044) (width 0.2) (layer "F.Cu") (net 4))
 (segment (start 119.11 90.631321) (end 116.34 87.861321) (width 0.2) (layer "F.Cu") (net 4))
 (segment (start 179.42 100) (end 179.42 94.2712) (width 0.2) (layer "F.Cu") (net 4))
 (segment (start 129.4892 94.0308) (end 129.4892 93.91) (width 0.2) (layer "F.Cu") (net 4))
 (segment (start 129.4892 93.91) (end 119.783654 93.91) (width 0.2) (layer "F.Cu") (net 4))
 (segment (start 179.7812 93.91) (end 177.5968 93.91) (width 0.2) (layer "F.Cu") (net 4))
 (segment (start 133.72 96.2324) (end 136.0424 93.91) (width 0.2) (layer "F.Cu") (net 4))
 (segment (start 119.783654 93.91) (end 119.11 93.236346) (width 0.2) (layer "F.Cu") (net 4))
 (segment (start 145.78 73.6252) (end 145.78 72) (width 0.2) (layer "F.Cu") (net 4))
 (segment (start 127.762 95.758) (end 129.4892 94.0308) (width 0.2) (layer "F.Cu") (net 4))
 (segment (start 162.6668 108.84) (end 177.5968 93.91) (width 0.2) (layer "F.Cu") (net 4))
 (segment (start 126.9 72.455635) (end 126.9 71.544365) (width 0.2) (layer "F.Cu") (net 4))
 (segment (start 184.101346 93.91) (end 179.7812 93.91) (width 0.2) (layer "F.Cu") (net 4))
 (segment (start 144.4756 73.3044) (end 145.78 72) (width 0.2) (layer "F.Cu") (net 4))
 (segment (start 153.0096 93.91) (end 136.0424 93.91) (width 0.2) (layer "F.Cu") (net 4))
 (segment (start 124.5 63.35) (end 134.3684 63.35) (width 0.2) (layer "F.Cu") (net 4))
 (segment (start 160.72 108.84) (end 162.6668 108.84) (width 0.2) (layer "F.Cu") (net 4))
 (segment (start 143.256 76.1492) (end 145.78 73.6252) (width 0.2) (layer "F.Cu") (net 4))
 (segment (start 122.3264 102.1536) (end 122.3264 99.8728) (width 0.2) (layer "F.Cu") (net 4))
 (segment (start 188.37 87.775) (end 188.37 89.641346) (width 0.2) (layer "F.Cu") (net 4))
 (segment (start 134.3684 63.35) (end 138.176 67.1576) (width 0.2) (layer "F.Cu") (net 4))
 (segment (start 117.72 106.76) (end 122.3264 102.1536) (width 0.2) (layer "F.Cu") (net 4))
 (segment (start 119.11 93.236346) (end 119.11 90.631321) (width 0.2) (layer "F.Cu") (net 4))
 (segment (start 128.455635 70.9) (end 129.44 71.884365) (width 0.2) (layer "F.Cu") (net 4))
 (via (at 122.3264 99.8728) (size 0.6) (drill 0.3) (layers "F.Cu" "B.Cu") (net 4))
 (via (at 138.176 67.1576) (size 0.6) (drill 0.3) (layers "F.Cu" "B.Cu") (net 4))
 (via (at 127.762 95.758) (size 0.6) (drill 0.3) (layers "F.Cu" "B.Cu") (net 4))
 (via (at 143.256 76.1492) (size 0.6) (drill 0.3) (layers "F.Cu" "B.Cu") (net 4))
 (segment (start 126.4412 95.758) (end 127.762 95.758) (width 0.2) (layer "B.Cu") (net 4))
 (segment (start 141.8 70.7816) (end 141.8 74.6932) (width 0.2) (layer "B.Cu") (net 4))
 (segment (start 122.3264 99.8728) (end 126.4412 95.758) (width 0.2) (layer "B.Cu") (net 4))
 (segment (start 138.176 67.1576) (end 141.8 70.7816) (width 0.2) (layer "B.Cu") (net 4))
 (segment (start 141.8 74.6932) (end 143.256 76.1492) (width 0.2) (layer "B.Cu") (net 4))
 (segment (start 187.22 71.385) (end 169.4002 89.2048) (width 0.2) (layer "F.Cu") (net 17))
 (segment (start 169.4002 89.2048) (end 120.7516 89.2048) (width 0.2) (layer "F.Cu") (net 17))
 (segment (start 120.7516 89.2048) (end 120.38 88.8332) (width 0.2) (layer "F.Cu") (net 17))
 (segment (start 120.38 88.8332) (end 120.38 87.24) (width 0.2) (layer "F.Cu") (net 17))
 (segment (start 188.77 74.915) (end 188.77 70.069315) (width 0.2) (layer "F.Cu") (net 14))
 (segment (start 188.77 70.069315) (end 188.449085 69.7484) (width 0.2) (layer "F.Cu") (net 14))
 (segment (start 122.6316 69.7484) (end 120.38 72) (width 0.2) (layer "F.Cu") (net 14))
 (segment (start 187.22 76.465) (end 188.77 74.915) (width 0.2) (layer "F.Cu") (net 14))
 (segment (start 188.449085 69.7484) (end 122.6316 69.7484) (width 0.2) (layer "F.Cu") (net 14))
 (segment (start 116.74 71.544365) (end 116.74 72.455635) (width 0.2) (layer "F.Cu") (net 13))
 (segment (start 117.784365 73.5) (end 121.42 73.5) (width 0.2) (layer "F.Cu") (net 13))
 (segment (start 116.74 72.455635) (end 117.784365 73.5) (width 0.2) (layer "F.Cu") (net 13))
 (segment (start 188.995686 68.9484) (end 119.335965 68.9484) (width 0.2) (layer "F.Cu") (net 13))
 (segment (start 189.57 81.735) (end 189.57 69.522714) (width 0.2) (layer "F.Cu") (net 13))
 (segment (start 121.42 73.5) (end 122.92 72) (width 0.2) (layer "F.Cu") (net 13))
 (segment (start 187.22 84.085) (end 189.57 81.735) (width 0.2) (layer "F.Cu") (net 13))
 (segment (start 119.335965 68.9484) (end 116.74 71.544365) (width 0.2) (layer "F.Cu") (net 13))
 (segment (start 189.57 69.522714) (end 188.995686 68.9484) (width 0.2) (layer "F.Cu") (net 13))
 (segment (start 187.22 81.545) (end 179.1602 89.6048) (width 0.2) (layer "F.Cu") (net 11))
 (segment (start 118.649165 89.6048) (end 116.74 87.695635) (width 0.2) (layer "F.Cu") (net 11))
 (segment (start 179.1602 89.6048) (end 118.649165 89.6048) (width 0.2) (layer "F.Cu") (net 11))
 (segment (start 116.74 83.26) (end 128 72) (width 0.2) (layer "F.Cu") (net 11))
 (segment (start 116.74 87.695635) (end 116.74 83.26) (width 0.2) (layer "F.Cu") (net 11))
 (segment (start 133.08 70.5264) (end 133.1468 70.4596) (width 0.2) (layer "F.Cu") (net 9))
 (segment (start 133.08 72) (end 133.08 70.5264) (width 0.2) (layer "F.Cu") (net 9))
 (segment (start 189.58 100) (end 187.48 100) (width 0.2) (layer "F.Cu") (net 9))
 (segment (start 187.48 100) (end 182.22 105.26) (width 0.2) (layer "F.Cu") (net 9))
 (via (at 133.1468 70.4596) (size 0.6) (drill 0.3) (layers "F.Cu" "B.Cu") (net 9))
 (segment (start 133.1468 70.4596) (end 137.0488 66.5576) (width 0.2) (layer "B.Cu") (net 9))
 (segment (start 137.0488 66.5576) (end 156.1376 66.5576) (width 0.2) (layer "B.Cu") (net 9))
 (segment (start 156.1376 66.5576) (end 189.58 100) (width 0.2) (layer "B.Cu") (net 9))
 (segment (start 159.385 97.765) (end 160.535 98.915) (width 0.2) (layer "F.Cu") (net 23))
 (segment (start 163.075 95.9682) (end 161.8488 94.742) (width 0.2) (layer "F.Cu") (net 23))
 (segment (start 162.684132 98.915) (end 163.075 98.524132) (width 0.2) (layer "F.Cu") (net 23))
 (segment (start 163.075 98.524132) (end 163.075 95.9682) (width 0.2) (layer "F.Cu") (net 23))
 (segment (start 160.535 98.915) (end 162.684132 98.915) (width 0.2) (layer "F.Cu") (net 23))
 (via (at 161.8488 94.742) (size 0.6) (drill 0.3) (layers "F.Cu" "B.Cu") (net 23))
 (segment (start 136.72 72.455635) (end 136.72 71.544365) (width 0.2) (layer "B.Cu") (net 23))
 (segment (start 161.8488 94.133165) (end 149.046435 81.3308) (width 0.2) (layer "B.Cu") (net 23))
 (segment (start 145.595165 81.3308) (end 136.72 72.455635) (width 0.2) (layer "B.Cu") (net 23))
 (segment (start 134.52 71.544365) (end 134.52 86.14) (width 0.2) (layer "B.Cu") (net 23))
 (segment (start 149.046435 81.3308) (end 145.595165 81.3308) (width 0.2) (layer "B.Cu") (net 23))
 (segment (start 161.8488 94.742) (end 161.8488 94.133165) (width 0.2) (layer "B.Cu") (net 23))
 (segment (start 135.164365 70.9) (end 134.52 71.544365) (width 0.2) (layer "B.Cu") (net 23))
 (segment (start 134.52 86.14) (end 135.62 87.24) (width 0.2) (layer "B.Cu") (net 23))
 (segment (start 136.075635 70.9) (end 135.164365 70.9) (width 0.2) (layer "B.Cu") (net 23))
 (segment (start 136.72 71.544365) (end 136.075635 70.9) (width 0.2) (layer "B.Cu") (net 23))
 (segment (start 116.174315 74.213515) (end 120.0404 78.0796) (width 0.2) (layer "F.Cu") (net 19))
 (segment (start 116.174315 66.675685) (end 116.174315 74.213515) (width 0.2) (layer "F.Cu") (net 19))
 (segment (start 119.5 63.35) (end 116.174315 66.675685) (width 0.2) (layer "F.Cu") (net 19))
 (via (at 120.0404 78.0796) (size 0.6) (drill 0.3) (layers "F.Cu" "B.Cu") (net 19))
 (segment (start 120.0404 78.0796) (end 125.46 83.4992) (width 0.2) (layer "B.Cu") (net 19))
 (segment (start 125.46 83.4992) (end 125.46 87.24) (width 0.2) (layer "B.Cu") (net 19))
 (segment (start 159.3596 95.1996) (end 159.3596 95.0468) (width 0.2) (layer "F.Cu") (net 24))
 (segment (start 161.925 97.765) (end 159.3596 95.1996) (width 0.2) (layer "F.Cu") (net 24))
 (via (at 159.3596 95.0468) (size 0.6) (drill 0.3) (layers "F.Cu" "B.Cu") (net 24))
 (segment (start 117.002 90.327871) (end 118.937871 88.392) (width 0.2) (layer "B.Cu") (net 24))
 (segment (start 137.008 88.392) (end 138.16 87.24) (width 0.2) (layer "B.Cu") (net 24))
 (segment (start 158.7088 95.6976) (end 145.1356 95.6976) (width 0.2) (layer "B.Cu") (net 24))
 (segment (start 159.3596 95.0468) (end 158.7088 95.6976) (width 0.2) (layer "B.Cu") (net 24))
 (segment (start 118.937871 88.392) (end 137.008 88.392) (width 0.2) (layer "B.Cu") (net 24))
 (segment (start 140.6144 91.1764) (end 117.353471 91.1764) (width 0.2) (layer "B.Cu") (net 24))
 (segment (start 117.353471 91.1764) (end 117.002 90.824929) (width 0.2) (layer "B.Cu") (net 24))
 (segment (start 145.1356 95.6976) (end 140.6144 91.1764) (width 0.2) (layer "B.Cu") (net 24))
 (segment (start 117.002 90.824929) (end 117.002 90.327871) (width 0.2) (layer "B.Cu") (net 24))
 (segment (start 117.243654 91.61) (end 117.897007 91.61) (width 0.2) (layer "F.Cu") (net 10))
 (segment (start 115.94 80.7068) (end 117.5004 79.1464) (width 0.2) (layer "F.Cu") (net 10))
 (segment (start 115.94 88.027007) (end 115.94 80.7068) (width 0.2) (layer "F.Cu") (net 10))
 (segment (start 122.9264 106.5536) (end 122.9264 99.592746) (width 0.2) (layer "F.Cu") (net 10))
 (segment (start 118.71 90.797007) (end 115.94 88.027007) (width 0.2) (layer "F.Cu") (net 10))
 (segment (start 117.897007 91.61) (end 118.71 90.797007) (width 0.2) (layer "F.Cu") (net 10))
 (segment (start 116.57 93.236346) (end 116.57 92.283654) (width 0.2) (layer "F.Cu") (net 10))
 (segment (start 116.57 92.283654) (end 117.243654 91.61) (width 0.2) (layer "F.Cu") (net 10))
 (segment (start 122.72 106.76) (end 122.9264 106.5536) (width 0.2) (layer "F.Cu") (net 10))
 (segment (start 122.9264 99.592746) (end 116.57 93.236346) (width 0.2) (layer "F.Cu") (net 10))
 (via (at 117.5004 79.1464) (size 0.6) (drill 0.3) (layers "F.Cu" "B.Cu") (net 10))
 (segment (start 125.0604 77.4796) (end 130.54 72) (width 0.2) (layer "B.Cu") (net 10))
 (segment (start 119.1672 77.4796) (end 125.0604 77.4796) (width 0.2) (layer "B.Cu") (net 10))
 (segment (start 117.5004 79.1464) (end 119.1672 77.4796) (width 0.2) (layer "B.Cu") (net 10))
 (segment (start 186.37 90.015) (end 123.005 90.015) (width 0.2) (layer "F.Cu") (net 31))
 (segment (start 123.005 90.015) (end 120.26 92.76) (width 0.2) (layer "F.Cu") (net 31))
 (segment (start 187.22 89.165) (end 186.37 90.015) (width 0.2) (layer "F.Cu") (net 31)))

